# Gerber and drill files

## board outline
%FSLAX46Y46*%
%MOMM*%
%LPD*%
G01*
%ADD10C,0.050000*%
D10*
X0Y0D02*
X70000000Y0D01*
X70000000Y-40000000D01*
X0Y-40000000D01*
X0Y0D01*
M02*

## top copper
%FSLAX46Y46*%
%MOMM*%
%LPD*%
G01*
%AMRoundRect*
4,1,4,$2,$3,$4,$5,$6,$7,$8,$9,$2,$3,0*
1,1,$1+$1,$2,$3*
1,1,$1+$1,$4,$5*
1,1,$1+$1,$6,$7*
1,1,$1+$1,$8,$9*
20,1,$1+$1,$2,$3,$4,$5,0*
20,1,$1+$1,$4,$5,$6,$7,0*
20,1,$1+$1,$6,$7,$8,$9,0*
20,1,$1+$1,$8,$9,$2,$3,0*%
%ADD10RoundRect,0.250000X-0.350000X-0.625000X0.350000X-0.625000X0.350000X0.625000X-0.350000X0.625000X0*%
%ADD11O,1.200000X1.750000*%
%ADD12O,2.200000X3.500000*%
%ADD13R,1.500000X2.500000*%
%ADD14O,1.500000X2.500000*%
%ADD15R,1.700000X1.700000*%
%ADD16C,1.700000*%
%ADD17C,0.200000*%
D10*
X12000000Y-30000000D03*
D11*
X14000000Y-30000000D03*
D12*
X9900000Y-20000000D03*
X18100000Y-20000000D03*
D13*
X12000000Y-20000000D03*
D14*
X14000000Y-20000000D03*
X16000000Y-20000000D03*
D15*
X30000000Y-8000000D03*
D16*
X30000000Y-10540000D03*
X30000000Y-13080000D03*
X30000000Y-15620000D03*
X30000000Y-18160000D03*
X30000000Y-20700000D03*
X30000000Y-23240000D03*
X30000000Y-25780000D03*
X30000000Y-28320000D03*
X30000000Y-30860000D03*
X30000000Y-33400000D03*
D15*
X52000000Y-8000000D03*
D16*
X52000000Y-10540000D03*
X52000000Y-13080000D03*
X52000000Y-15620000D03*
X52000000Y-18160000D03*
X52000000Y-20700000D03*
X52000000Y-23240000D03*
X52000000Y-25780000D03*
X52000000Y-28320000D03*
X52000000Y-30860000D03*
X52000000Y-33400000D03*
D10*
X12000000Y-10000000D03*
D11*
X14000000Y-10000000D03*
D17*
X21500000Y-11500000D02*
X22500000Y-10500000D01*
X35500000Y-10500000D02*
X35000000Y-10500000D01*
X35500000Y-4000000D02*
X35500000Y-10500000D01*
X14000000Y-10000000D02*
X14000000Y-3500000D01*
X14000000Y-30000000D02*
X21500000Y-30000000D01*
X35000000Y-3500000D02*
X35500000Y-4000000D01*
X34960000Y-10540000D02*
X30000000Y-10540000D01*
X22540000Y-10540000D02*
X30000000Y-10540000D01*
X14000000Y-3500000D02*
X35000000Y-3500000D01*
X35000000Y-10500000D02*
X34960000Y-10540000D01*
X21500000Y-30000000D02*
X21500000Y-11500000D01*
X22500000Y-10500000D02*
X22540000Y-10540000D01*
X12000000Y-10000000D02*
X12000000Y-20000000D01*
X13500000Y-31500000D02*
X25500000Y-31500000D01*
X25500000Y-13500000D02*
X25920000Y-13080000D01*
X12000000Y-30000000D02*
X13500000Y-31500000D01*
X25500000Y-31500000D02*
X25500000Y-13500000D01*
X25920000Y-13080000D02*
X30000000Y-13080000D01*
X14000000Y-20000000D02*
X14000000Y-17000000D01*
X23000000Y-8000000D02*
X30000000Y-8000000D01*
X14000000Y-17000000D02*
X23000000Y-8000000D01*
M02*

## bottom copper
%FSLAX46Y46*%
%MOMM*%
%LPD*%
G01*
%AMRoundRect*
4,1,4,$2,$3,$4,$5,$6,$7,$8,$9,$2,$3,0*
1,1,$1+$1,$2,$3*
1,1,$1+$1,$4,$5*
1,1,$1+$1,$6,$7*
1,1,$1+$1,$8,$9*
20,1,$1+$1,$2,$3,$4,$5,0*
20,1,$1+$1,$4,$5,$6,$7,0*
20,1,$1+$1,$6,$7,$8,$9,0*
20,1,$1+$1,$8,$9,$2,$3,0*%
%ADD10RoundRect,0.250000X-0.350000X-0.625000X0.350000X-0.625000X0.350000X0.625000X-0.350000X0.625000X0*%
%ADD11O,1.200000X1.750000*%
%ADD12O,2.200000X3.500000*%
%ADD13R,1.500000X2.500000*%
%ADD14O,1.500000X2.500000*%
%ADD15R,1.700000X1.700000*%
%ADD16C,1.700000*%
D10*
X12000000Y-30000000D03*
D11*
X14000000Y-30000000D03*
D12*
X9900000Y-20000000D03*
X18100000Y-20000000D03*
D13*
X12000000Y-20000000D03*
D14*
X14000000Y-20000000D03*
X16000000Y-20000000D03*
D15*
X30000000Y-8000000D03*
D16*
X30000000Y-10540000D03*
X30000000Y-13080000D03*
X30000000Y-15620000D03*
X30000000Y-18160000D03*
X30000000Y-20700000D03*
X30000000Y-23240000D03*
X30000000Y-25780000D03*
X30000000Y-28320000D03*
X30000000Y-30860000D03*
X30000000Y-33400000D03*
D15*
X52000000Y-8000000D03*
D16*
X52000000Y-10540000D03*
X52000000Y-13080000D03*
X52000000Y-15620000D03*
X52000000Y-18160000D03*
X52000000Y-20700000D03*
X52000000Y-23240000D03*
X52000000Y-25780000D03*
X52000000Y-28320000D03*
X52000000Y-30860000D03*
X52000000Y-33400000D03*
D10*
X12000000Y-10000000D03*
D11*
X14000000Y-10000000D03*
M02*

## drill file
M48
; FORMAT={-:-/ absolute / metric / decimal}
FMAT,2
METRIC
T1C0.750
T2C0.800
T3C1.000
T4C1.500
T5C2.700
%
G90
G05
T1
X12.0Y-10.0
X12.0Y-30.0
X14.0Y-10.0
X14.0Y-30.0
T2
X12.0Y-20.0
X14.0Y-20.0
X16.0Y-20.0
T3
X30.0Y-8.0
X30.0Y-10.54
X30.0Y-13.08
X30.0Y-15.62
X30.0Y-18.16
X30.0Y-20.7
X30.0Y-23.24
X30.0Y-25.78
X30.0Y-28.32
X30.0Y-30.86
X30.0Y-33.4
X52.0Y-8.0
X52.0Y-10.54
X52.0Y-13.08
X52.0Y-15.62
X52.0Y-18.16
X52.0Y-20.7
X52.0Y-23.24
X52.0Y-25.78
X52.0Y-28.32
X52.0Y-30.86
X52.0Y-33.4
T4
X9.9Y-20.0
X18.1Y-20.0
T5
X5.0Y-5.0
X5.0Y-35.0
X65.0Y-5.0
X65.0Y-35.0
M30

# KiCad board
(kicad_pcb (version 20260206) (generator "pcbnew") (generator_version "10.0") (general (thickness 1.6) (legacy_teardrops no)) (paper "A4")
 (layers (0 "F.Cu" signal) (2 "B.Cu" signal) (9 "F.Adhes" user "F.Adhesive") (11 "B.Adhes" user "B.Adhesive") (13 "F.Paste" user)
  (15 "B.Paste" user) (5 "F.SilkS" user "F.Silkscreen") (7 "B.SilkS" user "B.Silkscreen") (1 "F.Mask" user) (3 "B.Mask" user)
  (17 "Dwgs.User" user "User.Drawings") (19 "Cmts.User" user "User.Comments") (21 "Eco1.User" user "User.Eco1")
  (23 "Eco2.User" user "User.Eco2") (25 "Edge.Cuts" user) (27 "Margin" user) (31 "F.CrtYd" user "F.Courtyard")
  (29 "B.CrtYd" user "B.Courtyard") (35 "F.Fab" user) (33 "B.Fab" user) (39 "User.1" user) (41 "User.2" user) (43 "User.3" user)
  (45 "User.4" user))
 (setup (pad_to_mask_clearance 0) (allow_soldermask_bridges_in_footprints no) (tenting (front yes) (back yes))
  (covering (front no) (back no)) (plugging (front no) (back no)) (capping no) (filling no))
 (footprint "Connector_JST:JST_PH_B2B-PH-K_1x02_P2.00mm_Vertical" (layer "F.Cu") (at 12 30)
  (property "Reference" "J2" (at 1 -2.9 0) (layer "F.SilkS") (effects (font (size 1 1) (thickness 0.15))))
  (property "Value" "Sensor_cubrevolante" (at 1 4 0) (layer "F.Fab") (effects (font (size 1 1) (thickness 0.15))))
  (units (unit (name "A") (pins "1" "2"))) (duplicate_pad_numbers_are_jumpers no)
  (pad "1" thru_hole roundrect (at 0 0) (size 1.2 1.75) (drill 0.75) (layers "*.Cu" "*.Mask") (remove_unused_layers no)
   (roundrect_rratio 0.208333) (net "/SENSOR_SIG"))
  (pad "2" thru_hole oval (at 2 0) (size 1.2 1.75) (drill 0.75) (layers "*.Cu" "*.Mask") (remove_unused_layers no) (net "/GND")))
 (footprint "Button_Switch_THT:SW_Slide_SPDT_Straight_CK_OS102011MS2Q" (layer "F.Cu") (at 12 20)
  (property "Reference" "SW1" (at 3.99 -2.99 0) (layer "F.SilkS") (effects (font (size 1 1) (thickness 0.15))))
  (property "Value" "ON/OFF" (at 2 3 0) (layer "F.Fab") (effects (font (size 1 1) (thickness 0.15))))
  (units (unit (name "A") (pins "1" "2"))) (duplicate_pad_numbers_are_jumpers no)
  (pad "" thru_hole oval (at -2.1 0) (size 2.2 3.5) (drill 1.5) (layers "*.Cu" "*.Mask") (remove_unused_layers no))
  (pad "" thru_hole oval (at 6.1 0) (size 2.2 3.5) (drill 1.5) (layers "*.Cu" "*.Mask") (remove_unused_layers no))
  (pad "1" thru_hole rect (at 0 0) (size 1.5 2.5) (drill 0.8) (layers "*.Cu" "*.Mask") (remove_unused_layers no) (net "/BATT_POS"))
  (pad "2" thru_hole oval (at 2 0) (size 1.5 2.5) (drill 0.8) (layers "*.Cu" "*.Mask") (remove_unused_layers no) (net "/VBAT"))
  (pad "3" thru_hole oval (at 4 0) (size 1.5 2.5) (drill 0.8) (layers "*.Cu" "*.Mask") (remove_unused_layers no)))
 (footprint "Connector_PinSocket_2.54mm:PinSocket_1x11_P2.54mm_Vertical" (layer "F.Cu") (at 30 8)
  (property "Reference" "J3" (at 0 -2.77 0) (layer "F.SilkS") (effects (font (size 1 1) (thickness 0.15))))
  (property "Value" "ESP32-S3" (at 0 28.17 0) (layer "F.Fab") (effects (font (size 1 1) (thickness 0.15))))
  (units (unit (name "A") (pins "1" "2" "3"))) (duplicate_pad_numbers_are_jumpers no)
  (pad "1" thru_hole rect (at 0 0) (size 1.7 1.7) (drill 1) (layers "*.Cu" "*.Mask") (remove_unused_layers no) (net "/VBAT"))
  (pad "2" thru_hole circle (at 0 2.54) (size 1.7 1.7) (drill 1) (layers "*.Cu" "*.Mask") (remove_unused_layers no) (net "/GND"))
  (pad "3" thru_hole circle (at 0 5.08) (size 1.7 1.7) (drill 1) (layers "*.Cu" "*.Mask") (remove_unused_layers no) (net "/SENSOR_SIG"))
  (pad "4" thru_hole circle (at 0 7.62) (size 1.7 1.7) (drill 1) (layers "*.Cu" "*.Mask") (remove_unused_layers no))
  (pad "5" thru_hole circle (at 0 10.16) (size 1.7 1.7) (drill 1) (layers "*.Cu" "*.Mask") (remove_unused_layers no))
  (pad "6" thru_hole circle (at 0 12.7) (size 1.7 1.7) (drill 1) (layers "*.Cu" "*.Mask") (remove_unused_layers no))
  (pad "7" thru_hole circle (at 0 15.24) (size 1.7 1.7) (drill 1) (layers "*.Cu" "*.Mask") (remove_unused_layers no))
  (pad "8" thru_hole circle (at 0 17.78) (size 1.7 1.7) (drill 1) (layers "*.Cu" "*.Mask") (remove_unused_layers no))
  (pad "9" thru_hole circle (at 0 20.32) (size 1.7 1.7) (drill 1) (layers "*.Cu" "*.Mask") (remove_unused_layers no))
  (pad "10" thru_hole circle (at 0 22.86) (size 1.7 1.7) (drill 1) (layers "*.Cu" "*.Mask") (remove_unused_layers no))
  (pad "11" thru_hole circle (at 0 25.4) (size 1.7 1.7) (drill 1) (layers "*.Cu" "*.Mask") (remove_unused_layers no)))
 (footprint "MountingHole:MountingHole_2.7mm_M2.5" (layer "F.Cu") (at 65 35)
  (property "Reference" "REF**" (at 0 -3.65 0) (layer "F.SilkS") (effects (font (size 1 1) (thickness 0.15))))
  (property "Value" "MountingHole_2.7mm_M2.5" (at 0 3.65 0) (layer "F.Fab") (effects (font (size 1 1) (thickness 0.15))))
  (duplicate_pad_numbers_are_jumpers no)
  (pad "" np_thru_hole circle (at 0 0) (size 2.7 2.7) (drill 2.7) (layers "*.Cu" "*.Mask")))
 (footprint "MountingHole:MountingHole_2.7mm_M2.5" (layer "F.Cu") (at 65 5)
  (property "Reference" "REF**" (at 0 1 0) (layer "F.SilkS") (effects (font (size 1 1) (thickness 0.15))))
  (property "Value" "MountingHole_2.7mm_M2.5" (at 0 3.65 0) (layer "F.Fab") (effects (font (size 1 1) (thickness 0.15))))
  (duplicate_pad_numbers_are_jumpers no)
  (pad "" np_thru_hole circle (at 0 0) (size 2.7 2.7) (drill 2.7) (layers "*.Cu" "*.Mask")))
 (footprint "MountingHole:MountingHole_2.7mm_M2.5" (layer "F.Cu") (at 5 5)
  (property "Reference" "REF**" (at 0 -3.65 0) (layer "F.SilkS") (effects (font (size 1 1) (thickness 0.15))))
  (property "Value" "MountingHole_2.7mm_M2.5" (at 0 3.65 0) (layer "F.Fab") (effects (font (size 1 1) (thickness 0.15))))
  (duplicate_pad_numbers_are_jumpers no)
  (pad "" np_thru_hole circle (at 0 0) (size 2.7 2.7) (drill 2.7) (layers "*.Cu" "*.Mask")))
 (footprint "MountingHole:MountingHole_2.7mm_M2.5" (layer "F.Cu") (at 5 35)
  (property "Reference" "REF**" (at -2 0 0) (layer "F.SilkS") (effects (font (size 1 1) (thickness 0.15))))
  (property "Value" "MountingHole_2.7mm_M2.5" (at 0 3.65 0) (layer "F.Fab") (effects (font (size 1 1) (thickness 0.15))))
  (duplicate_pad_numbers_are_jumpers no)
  (pad "" np_thru_hole circle (at 0 0) (size 2.7 2.7) (drill 2.7) (layers "*.Cu" "*.Mask")))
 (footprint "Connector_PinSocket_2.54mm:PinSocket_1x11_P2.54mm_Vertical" (layer "F.Cu") (at 52 8)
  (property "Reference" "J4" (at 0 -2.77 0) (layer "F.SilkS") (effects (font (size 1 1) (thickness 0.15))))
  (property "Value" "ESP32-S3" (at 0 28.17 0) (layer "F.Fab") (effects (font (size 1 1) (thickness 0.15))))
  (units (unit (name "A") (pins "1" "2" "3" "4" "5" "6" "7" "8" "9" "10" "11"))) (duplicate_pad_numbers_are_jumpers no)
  (pad "1" thru_hole rect (at 0 0) (size 1.7 1.7) (drill 1) (layers "*.Cu" "*.Mask") (remove_unused_layers no)
   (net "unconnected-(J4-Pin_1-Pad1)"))
  (pad "2" thru_hole circle (at 0 2.54) (size 1.7 1.7) (drill 1) (layers "*.Cu" "*.Mask") (remove_unused_layers no)
   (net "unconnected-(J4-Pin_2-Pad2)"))
  (pad "3" thru_hole circle (at 0 5.08) (size 1.7 1.7) (drill 1) (layers "*.Cu" "*.Mask") (remove_unused_layers no)
   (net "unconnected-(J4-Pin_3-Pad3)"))
  (pad "4" thru_hole circle (at 0 7.62) (size 1.7 1.7) (drill 1) (layers "*.Cu" "*.Mask") (remove_unused_layers no)
   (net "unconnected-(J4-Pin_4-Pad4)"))
  (pad "5" thru_hole circle (at 0 10.16) (size 1.7 1.7) (drill 1) (layers "*.Cu" "*.Mask") (remove_unused_layers no)
   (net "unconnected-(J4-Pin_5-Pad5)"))
  (pad "6" thru_hole circle (at 0 12.7) (size 1.7 1.7) (drill 1) (layers "*.Cu" "*.Mask") (remove_unused_layers no)
   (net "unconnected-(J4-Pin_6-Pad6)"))
  (pad "7" thru_hole circle (at 0 15.24) (size 1.7 1.7) (drill 1) (layers "*.Cu" "*.Mask") (remove_unused_layers no)
   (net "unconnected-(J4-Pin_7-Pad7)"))
  (pad "8" thru_hole circle (at 0 17.78) (size 1.7 1.7) (drill 1) (layers "*.Cu" "*.Mask") (remove_unused_layers no)
   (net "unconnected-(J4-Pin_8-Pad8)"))
  (pad "9" thru_hole circle (at 0 20.32) (size 1.7 1.7) (drill 1) (layers "*.Cu" "*.Mask") (remove_unused_layers no)
   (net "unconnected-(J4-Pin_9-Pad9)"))
  (pad "10" thru_hole circle (at 0 22.86) (size 1.7 1.7) (drill 1) (layers "*.Cu" "*.Mask") (remove_unused_layers no)
   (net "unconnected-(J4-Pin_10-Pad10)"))
  (pad "11" thru_hole circle (at 0 25.4) (size 1.7 1.7) (drill 1) (layers "*.Cu" "*.Mask") (remove_unused_layers no)
   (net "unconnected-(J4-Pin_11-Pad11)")))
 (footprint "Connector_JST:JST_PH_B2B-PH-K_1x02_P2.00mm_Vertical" (layer "F.Cu") (at 12 10)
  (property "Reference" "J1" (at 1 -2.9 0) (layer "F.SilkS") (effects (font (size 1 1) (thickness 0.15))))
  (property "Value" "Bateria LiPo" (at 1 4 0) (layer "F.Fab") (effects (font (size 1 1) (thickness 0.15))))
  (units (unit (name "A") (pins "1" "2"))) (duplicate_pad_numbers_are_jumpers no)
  (pad "1" thru_hole roundrect (at 0 0) (size 1.2 1.75) (drill 0.75) (layers "*.Cu" "*.Mask") (remove_unused_layers no)
   (roundrect_rratio 0.208333) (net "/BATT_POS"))
  (pad "2" thru_hole oval (at 2 0) (size 1.2 1.75) (drill 0.75) (layers "*.Cu" "*.Mask") (remove_unused_layers no) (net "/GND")))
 (gr_rect (start 0 0) (end 70 40) (stroke (width 0.05) (type default)) (fill no) (layer "Edge.Cuts"))
 (segment (start 21.5 11.5) (end 22.5 10.5) (width 0.2) (layer "F.Cu") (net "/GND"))
 (segment (start 35.5 10.5) (end 35 10.5) (width 0.2) (layer "F.Cu") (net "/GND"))
 (segment (start 35.5 4) (end 35.5 10.5) (width 0.2) (layer "F.Cu") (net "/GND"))
 (segment (start 14 10) (end 14 3.5) (width 0.2) (layer "F.Cu") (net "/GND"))
 (segment (start 14 30) (end 21.5 30) (width 0.2) (layer "F.Cu") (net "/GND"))
 (segment (start 35 3.5) (end 35.5 4) (width 0.2) (layer "F.Cu") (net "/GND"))
 (segment (start 34.96 10.54) (end 30 10.54) (width 0.2) (layer "F.Cu") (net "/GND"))
 (segment (start 22.54 10.54) (end 30 10.54) (width 0.2) (layer "F.Cu") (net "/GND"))
 (segment (start 14 3.5) (end 35 3.5) (width 0.2) (layer "F.Cu") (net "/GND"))
 (segment (start 35 10.5) (end 34.96 10.54) (width 0.2) (layer "F.Cu") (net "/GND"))
 (segment (start 21.5 30) (end 21.5 11.5) (width 0.2) (layer "F.Cu") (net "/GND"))
 (segment (start 22.5 10.5) (end 22.54 10.54) (width 0.2) (layer "F.Cu") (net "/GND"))
 (segment (start 12 10) (end 12 20) (width 0.2) (layer "F.Cu") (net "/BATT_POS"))
 (segment (start 13.5 31.5) (end 25.5 31.5) (width 0.2) (layer "F.Cu") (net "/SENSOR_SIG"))
 (segment (start 25.5 13.5) (end 25.92 13.08) (width 0.2) (layer "F.Cu") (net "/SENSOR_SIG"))
 (segment (start 12 30) (end 13.5 31.5) (width 0.2) (layer "F.Cu") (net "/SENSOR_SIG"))
 (segment (start 25.5 31.5) (end 25.5 13.5) (width 0.2) (layer "F.Cu") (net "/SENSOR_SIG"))
 (segment (start 25.92 13.08) (end 30 13.08) (width 0.2) (layer "F.Cu") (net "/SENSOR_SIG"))
 (segment (start 14 20) (end 14 17) (width 0.2) (layer "F.Cu") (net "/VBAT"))
 (segment (start 23 8) (end 30 8) (width 0.2) (layer "F.Cu") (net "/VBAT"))
 (segment (start 14 17) (end 23 8) (width 0.2) (layer "F.Cu") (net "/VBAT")))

